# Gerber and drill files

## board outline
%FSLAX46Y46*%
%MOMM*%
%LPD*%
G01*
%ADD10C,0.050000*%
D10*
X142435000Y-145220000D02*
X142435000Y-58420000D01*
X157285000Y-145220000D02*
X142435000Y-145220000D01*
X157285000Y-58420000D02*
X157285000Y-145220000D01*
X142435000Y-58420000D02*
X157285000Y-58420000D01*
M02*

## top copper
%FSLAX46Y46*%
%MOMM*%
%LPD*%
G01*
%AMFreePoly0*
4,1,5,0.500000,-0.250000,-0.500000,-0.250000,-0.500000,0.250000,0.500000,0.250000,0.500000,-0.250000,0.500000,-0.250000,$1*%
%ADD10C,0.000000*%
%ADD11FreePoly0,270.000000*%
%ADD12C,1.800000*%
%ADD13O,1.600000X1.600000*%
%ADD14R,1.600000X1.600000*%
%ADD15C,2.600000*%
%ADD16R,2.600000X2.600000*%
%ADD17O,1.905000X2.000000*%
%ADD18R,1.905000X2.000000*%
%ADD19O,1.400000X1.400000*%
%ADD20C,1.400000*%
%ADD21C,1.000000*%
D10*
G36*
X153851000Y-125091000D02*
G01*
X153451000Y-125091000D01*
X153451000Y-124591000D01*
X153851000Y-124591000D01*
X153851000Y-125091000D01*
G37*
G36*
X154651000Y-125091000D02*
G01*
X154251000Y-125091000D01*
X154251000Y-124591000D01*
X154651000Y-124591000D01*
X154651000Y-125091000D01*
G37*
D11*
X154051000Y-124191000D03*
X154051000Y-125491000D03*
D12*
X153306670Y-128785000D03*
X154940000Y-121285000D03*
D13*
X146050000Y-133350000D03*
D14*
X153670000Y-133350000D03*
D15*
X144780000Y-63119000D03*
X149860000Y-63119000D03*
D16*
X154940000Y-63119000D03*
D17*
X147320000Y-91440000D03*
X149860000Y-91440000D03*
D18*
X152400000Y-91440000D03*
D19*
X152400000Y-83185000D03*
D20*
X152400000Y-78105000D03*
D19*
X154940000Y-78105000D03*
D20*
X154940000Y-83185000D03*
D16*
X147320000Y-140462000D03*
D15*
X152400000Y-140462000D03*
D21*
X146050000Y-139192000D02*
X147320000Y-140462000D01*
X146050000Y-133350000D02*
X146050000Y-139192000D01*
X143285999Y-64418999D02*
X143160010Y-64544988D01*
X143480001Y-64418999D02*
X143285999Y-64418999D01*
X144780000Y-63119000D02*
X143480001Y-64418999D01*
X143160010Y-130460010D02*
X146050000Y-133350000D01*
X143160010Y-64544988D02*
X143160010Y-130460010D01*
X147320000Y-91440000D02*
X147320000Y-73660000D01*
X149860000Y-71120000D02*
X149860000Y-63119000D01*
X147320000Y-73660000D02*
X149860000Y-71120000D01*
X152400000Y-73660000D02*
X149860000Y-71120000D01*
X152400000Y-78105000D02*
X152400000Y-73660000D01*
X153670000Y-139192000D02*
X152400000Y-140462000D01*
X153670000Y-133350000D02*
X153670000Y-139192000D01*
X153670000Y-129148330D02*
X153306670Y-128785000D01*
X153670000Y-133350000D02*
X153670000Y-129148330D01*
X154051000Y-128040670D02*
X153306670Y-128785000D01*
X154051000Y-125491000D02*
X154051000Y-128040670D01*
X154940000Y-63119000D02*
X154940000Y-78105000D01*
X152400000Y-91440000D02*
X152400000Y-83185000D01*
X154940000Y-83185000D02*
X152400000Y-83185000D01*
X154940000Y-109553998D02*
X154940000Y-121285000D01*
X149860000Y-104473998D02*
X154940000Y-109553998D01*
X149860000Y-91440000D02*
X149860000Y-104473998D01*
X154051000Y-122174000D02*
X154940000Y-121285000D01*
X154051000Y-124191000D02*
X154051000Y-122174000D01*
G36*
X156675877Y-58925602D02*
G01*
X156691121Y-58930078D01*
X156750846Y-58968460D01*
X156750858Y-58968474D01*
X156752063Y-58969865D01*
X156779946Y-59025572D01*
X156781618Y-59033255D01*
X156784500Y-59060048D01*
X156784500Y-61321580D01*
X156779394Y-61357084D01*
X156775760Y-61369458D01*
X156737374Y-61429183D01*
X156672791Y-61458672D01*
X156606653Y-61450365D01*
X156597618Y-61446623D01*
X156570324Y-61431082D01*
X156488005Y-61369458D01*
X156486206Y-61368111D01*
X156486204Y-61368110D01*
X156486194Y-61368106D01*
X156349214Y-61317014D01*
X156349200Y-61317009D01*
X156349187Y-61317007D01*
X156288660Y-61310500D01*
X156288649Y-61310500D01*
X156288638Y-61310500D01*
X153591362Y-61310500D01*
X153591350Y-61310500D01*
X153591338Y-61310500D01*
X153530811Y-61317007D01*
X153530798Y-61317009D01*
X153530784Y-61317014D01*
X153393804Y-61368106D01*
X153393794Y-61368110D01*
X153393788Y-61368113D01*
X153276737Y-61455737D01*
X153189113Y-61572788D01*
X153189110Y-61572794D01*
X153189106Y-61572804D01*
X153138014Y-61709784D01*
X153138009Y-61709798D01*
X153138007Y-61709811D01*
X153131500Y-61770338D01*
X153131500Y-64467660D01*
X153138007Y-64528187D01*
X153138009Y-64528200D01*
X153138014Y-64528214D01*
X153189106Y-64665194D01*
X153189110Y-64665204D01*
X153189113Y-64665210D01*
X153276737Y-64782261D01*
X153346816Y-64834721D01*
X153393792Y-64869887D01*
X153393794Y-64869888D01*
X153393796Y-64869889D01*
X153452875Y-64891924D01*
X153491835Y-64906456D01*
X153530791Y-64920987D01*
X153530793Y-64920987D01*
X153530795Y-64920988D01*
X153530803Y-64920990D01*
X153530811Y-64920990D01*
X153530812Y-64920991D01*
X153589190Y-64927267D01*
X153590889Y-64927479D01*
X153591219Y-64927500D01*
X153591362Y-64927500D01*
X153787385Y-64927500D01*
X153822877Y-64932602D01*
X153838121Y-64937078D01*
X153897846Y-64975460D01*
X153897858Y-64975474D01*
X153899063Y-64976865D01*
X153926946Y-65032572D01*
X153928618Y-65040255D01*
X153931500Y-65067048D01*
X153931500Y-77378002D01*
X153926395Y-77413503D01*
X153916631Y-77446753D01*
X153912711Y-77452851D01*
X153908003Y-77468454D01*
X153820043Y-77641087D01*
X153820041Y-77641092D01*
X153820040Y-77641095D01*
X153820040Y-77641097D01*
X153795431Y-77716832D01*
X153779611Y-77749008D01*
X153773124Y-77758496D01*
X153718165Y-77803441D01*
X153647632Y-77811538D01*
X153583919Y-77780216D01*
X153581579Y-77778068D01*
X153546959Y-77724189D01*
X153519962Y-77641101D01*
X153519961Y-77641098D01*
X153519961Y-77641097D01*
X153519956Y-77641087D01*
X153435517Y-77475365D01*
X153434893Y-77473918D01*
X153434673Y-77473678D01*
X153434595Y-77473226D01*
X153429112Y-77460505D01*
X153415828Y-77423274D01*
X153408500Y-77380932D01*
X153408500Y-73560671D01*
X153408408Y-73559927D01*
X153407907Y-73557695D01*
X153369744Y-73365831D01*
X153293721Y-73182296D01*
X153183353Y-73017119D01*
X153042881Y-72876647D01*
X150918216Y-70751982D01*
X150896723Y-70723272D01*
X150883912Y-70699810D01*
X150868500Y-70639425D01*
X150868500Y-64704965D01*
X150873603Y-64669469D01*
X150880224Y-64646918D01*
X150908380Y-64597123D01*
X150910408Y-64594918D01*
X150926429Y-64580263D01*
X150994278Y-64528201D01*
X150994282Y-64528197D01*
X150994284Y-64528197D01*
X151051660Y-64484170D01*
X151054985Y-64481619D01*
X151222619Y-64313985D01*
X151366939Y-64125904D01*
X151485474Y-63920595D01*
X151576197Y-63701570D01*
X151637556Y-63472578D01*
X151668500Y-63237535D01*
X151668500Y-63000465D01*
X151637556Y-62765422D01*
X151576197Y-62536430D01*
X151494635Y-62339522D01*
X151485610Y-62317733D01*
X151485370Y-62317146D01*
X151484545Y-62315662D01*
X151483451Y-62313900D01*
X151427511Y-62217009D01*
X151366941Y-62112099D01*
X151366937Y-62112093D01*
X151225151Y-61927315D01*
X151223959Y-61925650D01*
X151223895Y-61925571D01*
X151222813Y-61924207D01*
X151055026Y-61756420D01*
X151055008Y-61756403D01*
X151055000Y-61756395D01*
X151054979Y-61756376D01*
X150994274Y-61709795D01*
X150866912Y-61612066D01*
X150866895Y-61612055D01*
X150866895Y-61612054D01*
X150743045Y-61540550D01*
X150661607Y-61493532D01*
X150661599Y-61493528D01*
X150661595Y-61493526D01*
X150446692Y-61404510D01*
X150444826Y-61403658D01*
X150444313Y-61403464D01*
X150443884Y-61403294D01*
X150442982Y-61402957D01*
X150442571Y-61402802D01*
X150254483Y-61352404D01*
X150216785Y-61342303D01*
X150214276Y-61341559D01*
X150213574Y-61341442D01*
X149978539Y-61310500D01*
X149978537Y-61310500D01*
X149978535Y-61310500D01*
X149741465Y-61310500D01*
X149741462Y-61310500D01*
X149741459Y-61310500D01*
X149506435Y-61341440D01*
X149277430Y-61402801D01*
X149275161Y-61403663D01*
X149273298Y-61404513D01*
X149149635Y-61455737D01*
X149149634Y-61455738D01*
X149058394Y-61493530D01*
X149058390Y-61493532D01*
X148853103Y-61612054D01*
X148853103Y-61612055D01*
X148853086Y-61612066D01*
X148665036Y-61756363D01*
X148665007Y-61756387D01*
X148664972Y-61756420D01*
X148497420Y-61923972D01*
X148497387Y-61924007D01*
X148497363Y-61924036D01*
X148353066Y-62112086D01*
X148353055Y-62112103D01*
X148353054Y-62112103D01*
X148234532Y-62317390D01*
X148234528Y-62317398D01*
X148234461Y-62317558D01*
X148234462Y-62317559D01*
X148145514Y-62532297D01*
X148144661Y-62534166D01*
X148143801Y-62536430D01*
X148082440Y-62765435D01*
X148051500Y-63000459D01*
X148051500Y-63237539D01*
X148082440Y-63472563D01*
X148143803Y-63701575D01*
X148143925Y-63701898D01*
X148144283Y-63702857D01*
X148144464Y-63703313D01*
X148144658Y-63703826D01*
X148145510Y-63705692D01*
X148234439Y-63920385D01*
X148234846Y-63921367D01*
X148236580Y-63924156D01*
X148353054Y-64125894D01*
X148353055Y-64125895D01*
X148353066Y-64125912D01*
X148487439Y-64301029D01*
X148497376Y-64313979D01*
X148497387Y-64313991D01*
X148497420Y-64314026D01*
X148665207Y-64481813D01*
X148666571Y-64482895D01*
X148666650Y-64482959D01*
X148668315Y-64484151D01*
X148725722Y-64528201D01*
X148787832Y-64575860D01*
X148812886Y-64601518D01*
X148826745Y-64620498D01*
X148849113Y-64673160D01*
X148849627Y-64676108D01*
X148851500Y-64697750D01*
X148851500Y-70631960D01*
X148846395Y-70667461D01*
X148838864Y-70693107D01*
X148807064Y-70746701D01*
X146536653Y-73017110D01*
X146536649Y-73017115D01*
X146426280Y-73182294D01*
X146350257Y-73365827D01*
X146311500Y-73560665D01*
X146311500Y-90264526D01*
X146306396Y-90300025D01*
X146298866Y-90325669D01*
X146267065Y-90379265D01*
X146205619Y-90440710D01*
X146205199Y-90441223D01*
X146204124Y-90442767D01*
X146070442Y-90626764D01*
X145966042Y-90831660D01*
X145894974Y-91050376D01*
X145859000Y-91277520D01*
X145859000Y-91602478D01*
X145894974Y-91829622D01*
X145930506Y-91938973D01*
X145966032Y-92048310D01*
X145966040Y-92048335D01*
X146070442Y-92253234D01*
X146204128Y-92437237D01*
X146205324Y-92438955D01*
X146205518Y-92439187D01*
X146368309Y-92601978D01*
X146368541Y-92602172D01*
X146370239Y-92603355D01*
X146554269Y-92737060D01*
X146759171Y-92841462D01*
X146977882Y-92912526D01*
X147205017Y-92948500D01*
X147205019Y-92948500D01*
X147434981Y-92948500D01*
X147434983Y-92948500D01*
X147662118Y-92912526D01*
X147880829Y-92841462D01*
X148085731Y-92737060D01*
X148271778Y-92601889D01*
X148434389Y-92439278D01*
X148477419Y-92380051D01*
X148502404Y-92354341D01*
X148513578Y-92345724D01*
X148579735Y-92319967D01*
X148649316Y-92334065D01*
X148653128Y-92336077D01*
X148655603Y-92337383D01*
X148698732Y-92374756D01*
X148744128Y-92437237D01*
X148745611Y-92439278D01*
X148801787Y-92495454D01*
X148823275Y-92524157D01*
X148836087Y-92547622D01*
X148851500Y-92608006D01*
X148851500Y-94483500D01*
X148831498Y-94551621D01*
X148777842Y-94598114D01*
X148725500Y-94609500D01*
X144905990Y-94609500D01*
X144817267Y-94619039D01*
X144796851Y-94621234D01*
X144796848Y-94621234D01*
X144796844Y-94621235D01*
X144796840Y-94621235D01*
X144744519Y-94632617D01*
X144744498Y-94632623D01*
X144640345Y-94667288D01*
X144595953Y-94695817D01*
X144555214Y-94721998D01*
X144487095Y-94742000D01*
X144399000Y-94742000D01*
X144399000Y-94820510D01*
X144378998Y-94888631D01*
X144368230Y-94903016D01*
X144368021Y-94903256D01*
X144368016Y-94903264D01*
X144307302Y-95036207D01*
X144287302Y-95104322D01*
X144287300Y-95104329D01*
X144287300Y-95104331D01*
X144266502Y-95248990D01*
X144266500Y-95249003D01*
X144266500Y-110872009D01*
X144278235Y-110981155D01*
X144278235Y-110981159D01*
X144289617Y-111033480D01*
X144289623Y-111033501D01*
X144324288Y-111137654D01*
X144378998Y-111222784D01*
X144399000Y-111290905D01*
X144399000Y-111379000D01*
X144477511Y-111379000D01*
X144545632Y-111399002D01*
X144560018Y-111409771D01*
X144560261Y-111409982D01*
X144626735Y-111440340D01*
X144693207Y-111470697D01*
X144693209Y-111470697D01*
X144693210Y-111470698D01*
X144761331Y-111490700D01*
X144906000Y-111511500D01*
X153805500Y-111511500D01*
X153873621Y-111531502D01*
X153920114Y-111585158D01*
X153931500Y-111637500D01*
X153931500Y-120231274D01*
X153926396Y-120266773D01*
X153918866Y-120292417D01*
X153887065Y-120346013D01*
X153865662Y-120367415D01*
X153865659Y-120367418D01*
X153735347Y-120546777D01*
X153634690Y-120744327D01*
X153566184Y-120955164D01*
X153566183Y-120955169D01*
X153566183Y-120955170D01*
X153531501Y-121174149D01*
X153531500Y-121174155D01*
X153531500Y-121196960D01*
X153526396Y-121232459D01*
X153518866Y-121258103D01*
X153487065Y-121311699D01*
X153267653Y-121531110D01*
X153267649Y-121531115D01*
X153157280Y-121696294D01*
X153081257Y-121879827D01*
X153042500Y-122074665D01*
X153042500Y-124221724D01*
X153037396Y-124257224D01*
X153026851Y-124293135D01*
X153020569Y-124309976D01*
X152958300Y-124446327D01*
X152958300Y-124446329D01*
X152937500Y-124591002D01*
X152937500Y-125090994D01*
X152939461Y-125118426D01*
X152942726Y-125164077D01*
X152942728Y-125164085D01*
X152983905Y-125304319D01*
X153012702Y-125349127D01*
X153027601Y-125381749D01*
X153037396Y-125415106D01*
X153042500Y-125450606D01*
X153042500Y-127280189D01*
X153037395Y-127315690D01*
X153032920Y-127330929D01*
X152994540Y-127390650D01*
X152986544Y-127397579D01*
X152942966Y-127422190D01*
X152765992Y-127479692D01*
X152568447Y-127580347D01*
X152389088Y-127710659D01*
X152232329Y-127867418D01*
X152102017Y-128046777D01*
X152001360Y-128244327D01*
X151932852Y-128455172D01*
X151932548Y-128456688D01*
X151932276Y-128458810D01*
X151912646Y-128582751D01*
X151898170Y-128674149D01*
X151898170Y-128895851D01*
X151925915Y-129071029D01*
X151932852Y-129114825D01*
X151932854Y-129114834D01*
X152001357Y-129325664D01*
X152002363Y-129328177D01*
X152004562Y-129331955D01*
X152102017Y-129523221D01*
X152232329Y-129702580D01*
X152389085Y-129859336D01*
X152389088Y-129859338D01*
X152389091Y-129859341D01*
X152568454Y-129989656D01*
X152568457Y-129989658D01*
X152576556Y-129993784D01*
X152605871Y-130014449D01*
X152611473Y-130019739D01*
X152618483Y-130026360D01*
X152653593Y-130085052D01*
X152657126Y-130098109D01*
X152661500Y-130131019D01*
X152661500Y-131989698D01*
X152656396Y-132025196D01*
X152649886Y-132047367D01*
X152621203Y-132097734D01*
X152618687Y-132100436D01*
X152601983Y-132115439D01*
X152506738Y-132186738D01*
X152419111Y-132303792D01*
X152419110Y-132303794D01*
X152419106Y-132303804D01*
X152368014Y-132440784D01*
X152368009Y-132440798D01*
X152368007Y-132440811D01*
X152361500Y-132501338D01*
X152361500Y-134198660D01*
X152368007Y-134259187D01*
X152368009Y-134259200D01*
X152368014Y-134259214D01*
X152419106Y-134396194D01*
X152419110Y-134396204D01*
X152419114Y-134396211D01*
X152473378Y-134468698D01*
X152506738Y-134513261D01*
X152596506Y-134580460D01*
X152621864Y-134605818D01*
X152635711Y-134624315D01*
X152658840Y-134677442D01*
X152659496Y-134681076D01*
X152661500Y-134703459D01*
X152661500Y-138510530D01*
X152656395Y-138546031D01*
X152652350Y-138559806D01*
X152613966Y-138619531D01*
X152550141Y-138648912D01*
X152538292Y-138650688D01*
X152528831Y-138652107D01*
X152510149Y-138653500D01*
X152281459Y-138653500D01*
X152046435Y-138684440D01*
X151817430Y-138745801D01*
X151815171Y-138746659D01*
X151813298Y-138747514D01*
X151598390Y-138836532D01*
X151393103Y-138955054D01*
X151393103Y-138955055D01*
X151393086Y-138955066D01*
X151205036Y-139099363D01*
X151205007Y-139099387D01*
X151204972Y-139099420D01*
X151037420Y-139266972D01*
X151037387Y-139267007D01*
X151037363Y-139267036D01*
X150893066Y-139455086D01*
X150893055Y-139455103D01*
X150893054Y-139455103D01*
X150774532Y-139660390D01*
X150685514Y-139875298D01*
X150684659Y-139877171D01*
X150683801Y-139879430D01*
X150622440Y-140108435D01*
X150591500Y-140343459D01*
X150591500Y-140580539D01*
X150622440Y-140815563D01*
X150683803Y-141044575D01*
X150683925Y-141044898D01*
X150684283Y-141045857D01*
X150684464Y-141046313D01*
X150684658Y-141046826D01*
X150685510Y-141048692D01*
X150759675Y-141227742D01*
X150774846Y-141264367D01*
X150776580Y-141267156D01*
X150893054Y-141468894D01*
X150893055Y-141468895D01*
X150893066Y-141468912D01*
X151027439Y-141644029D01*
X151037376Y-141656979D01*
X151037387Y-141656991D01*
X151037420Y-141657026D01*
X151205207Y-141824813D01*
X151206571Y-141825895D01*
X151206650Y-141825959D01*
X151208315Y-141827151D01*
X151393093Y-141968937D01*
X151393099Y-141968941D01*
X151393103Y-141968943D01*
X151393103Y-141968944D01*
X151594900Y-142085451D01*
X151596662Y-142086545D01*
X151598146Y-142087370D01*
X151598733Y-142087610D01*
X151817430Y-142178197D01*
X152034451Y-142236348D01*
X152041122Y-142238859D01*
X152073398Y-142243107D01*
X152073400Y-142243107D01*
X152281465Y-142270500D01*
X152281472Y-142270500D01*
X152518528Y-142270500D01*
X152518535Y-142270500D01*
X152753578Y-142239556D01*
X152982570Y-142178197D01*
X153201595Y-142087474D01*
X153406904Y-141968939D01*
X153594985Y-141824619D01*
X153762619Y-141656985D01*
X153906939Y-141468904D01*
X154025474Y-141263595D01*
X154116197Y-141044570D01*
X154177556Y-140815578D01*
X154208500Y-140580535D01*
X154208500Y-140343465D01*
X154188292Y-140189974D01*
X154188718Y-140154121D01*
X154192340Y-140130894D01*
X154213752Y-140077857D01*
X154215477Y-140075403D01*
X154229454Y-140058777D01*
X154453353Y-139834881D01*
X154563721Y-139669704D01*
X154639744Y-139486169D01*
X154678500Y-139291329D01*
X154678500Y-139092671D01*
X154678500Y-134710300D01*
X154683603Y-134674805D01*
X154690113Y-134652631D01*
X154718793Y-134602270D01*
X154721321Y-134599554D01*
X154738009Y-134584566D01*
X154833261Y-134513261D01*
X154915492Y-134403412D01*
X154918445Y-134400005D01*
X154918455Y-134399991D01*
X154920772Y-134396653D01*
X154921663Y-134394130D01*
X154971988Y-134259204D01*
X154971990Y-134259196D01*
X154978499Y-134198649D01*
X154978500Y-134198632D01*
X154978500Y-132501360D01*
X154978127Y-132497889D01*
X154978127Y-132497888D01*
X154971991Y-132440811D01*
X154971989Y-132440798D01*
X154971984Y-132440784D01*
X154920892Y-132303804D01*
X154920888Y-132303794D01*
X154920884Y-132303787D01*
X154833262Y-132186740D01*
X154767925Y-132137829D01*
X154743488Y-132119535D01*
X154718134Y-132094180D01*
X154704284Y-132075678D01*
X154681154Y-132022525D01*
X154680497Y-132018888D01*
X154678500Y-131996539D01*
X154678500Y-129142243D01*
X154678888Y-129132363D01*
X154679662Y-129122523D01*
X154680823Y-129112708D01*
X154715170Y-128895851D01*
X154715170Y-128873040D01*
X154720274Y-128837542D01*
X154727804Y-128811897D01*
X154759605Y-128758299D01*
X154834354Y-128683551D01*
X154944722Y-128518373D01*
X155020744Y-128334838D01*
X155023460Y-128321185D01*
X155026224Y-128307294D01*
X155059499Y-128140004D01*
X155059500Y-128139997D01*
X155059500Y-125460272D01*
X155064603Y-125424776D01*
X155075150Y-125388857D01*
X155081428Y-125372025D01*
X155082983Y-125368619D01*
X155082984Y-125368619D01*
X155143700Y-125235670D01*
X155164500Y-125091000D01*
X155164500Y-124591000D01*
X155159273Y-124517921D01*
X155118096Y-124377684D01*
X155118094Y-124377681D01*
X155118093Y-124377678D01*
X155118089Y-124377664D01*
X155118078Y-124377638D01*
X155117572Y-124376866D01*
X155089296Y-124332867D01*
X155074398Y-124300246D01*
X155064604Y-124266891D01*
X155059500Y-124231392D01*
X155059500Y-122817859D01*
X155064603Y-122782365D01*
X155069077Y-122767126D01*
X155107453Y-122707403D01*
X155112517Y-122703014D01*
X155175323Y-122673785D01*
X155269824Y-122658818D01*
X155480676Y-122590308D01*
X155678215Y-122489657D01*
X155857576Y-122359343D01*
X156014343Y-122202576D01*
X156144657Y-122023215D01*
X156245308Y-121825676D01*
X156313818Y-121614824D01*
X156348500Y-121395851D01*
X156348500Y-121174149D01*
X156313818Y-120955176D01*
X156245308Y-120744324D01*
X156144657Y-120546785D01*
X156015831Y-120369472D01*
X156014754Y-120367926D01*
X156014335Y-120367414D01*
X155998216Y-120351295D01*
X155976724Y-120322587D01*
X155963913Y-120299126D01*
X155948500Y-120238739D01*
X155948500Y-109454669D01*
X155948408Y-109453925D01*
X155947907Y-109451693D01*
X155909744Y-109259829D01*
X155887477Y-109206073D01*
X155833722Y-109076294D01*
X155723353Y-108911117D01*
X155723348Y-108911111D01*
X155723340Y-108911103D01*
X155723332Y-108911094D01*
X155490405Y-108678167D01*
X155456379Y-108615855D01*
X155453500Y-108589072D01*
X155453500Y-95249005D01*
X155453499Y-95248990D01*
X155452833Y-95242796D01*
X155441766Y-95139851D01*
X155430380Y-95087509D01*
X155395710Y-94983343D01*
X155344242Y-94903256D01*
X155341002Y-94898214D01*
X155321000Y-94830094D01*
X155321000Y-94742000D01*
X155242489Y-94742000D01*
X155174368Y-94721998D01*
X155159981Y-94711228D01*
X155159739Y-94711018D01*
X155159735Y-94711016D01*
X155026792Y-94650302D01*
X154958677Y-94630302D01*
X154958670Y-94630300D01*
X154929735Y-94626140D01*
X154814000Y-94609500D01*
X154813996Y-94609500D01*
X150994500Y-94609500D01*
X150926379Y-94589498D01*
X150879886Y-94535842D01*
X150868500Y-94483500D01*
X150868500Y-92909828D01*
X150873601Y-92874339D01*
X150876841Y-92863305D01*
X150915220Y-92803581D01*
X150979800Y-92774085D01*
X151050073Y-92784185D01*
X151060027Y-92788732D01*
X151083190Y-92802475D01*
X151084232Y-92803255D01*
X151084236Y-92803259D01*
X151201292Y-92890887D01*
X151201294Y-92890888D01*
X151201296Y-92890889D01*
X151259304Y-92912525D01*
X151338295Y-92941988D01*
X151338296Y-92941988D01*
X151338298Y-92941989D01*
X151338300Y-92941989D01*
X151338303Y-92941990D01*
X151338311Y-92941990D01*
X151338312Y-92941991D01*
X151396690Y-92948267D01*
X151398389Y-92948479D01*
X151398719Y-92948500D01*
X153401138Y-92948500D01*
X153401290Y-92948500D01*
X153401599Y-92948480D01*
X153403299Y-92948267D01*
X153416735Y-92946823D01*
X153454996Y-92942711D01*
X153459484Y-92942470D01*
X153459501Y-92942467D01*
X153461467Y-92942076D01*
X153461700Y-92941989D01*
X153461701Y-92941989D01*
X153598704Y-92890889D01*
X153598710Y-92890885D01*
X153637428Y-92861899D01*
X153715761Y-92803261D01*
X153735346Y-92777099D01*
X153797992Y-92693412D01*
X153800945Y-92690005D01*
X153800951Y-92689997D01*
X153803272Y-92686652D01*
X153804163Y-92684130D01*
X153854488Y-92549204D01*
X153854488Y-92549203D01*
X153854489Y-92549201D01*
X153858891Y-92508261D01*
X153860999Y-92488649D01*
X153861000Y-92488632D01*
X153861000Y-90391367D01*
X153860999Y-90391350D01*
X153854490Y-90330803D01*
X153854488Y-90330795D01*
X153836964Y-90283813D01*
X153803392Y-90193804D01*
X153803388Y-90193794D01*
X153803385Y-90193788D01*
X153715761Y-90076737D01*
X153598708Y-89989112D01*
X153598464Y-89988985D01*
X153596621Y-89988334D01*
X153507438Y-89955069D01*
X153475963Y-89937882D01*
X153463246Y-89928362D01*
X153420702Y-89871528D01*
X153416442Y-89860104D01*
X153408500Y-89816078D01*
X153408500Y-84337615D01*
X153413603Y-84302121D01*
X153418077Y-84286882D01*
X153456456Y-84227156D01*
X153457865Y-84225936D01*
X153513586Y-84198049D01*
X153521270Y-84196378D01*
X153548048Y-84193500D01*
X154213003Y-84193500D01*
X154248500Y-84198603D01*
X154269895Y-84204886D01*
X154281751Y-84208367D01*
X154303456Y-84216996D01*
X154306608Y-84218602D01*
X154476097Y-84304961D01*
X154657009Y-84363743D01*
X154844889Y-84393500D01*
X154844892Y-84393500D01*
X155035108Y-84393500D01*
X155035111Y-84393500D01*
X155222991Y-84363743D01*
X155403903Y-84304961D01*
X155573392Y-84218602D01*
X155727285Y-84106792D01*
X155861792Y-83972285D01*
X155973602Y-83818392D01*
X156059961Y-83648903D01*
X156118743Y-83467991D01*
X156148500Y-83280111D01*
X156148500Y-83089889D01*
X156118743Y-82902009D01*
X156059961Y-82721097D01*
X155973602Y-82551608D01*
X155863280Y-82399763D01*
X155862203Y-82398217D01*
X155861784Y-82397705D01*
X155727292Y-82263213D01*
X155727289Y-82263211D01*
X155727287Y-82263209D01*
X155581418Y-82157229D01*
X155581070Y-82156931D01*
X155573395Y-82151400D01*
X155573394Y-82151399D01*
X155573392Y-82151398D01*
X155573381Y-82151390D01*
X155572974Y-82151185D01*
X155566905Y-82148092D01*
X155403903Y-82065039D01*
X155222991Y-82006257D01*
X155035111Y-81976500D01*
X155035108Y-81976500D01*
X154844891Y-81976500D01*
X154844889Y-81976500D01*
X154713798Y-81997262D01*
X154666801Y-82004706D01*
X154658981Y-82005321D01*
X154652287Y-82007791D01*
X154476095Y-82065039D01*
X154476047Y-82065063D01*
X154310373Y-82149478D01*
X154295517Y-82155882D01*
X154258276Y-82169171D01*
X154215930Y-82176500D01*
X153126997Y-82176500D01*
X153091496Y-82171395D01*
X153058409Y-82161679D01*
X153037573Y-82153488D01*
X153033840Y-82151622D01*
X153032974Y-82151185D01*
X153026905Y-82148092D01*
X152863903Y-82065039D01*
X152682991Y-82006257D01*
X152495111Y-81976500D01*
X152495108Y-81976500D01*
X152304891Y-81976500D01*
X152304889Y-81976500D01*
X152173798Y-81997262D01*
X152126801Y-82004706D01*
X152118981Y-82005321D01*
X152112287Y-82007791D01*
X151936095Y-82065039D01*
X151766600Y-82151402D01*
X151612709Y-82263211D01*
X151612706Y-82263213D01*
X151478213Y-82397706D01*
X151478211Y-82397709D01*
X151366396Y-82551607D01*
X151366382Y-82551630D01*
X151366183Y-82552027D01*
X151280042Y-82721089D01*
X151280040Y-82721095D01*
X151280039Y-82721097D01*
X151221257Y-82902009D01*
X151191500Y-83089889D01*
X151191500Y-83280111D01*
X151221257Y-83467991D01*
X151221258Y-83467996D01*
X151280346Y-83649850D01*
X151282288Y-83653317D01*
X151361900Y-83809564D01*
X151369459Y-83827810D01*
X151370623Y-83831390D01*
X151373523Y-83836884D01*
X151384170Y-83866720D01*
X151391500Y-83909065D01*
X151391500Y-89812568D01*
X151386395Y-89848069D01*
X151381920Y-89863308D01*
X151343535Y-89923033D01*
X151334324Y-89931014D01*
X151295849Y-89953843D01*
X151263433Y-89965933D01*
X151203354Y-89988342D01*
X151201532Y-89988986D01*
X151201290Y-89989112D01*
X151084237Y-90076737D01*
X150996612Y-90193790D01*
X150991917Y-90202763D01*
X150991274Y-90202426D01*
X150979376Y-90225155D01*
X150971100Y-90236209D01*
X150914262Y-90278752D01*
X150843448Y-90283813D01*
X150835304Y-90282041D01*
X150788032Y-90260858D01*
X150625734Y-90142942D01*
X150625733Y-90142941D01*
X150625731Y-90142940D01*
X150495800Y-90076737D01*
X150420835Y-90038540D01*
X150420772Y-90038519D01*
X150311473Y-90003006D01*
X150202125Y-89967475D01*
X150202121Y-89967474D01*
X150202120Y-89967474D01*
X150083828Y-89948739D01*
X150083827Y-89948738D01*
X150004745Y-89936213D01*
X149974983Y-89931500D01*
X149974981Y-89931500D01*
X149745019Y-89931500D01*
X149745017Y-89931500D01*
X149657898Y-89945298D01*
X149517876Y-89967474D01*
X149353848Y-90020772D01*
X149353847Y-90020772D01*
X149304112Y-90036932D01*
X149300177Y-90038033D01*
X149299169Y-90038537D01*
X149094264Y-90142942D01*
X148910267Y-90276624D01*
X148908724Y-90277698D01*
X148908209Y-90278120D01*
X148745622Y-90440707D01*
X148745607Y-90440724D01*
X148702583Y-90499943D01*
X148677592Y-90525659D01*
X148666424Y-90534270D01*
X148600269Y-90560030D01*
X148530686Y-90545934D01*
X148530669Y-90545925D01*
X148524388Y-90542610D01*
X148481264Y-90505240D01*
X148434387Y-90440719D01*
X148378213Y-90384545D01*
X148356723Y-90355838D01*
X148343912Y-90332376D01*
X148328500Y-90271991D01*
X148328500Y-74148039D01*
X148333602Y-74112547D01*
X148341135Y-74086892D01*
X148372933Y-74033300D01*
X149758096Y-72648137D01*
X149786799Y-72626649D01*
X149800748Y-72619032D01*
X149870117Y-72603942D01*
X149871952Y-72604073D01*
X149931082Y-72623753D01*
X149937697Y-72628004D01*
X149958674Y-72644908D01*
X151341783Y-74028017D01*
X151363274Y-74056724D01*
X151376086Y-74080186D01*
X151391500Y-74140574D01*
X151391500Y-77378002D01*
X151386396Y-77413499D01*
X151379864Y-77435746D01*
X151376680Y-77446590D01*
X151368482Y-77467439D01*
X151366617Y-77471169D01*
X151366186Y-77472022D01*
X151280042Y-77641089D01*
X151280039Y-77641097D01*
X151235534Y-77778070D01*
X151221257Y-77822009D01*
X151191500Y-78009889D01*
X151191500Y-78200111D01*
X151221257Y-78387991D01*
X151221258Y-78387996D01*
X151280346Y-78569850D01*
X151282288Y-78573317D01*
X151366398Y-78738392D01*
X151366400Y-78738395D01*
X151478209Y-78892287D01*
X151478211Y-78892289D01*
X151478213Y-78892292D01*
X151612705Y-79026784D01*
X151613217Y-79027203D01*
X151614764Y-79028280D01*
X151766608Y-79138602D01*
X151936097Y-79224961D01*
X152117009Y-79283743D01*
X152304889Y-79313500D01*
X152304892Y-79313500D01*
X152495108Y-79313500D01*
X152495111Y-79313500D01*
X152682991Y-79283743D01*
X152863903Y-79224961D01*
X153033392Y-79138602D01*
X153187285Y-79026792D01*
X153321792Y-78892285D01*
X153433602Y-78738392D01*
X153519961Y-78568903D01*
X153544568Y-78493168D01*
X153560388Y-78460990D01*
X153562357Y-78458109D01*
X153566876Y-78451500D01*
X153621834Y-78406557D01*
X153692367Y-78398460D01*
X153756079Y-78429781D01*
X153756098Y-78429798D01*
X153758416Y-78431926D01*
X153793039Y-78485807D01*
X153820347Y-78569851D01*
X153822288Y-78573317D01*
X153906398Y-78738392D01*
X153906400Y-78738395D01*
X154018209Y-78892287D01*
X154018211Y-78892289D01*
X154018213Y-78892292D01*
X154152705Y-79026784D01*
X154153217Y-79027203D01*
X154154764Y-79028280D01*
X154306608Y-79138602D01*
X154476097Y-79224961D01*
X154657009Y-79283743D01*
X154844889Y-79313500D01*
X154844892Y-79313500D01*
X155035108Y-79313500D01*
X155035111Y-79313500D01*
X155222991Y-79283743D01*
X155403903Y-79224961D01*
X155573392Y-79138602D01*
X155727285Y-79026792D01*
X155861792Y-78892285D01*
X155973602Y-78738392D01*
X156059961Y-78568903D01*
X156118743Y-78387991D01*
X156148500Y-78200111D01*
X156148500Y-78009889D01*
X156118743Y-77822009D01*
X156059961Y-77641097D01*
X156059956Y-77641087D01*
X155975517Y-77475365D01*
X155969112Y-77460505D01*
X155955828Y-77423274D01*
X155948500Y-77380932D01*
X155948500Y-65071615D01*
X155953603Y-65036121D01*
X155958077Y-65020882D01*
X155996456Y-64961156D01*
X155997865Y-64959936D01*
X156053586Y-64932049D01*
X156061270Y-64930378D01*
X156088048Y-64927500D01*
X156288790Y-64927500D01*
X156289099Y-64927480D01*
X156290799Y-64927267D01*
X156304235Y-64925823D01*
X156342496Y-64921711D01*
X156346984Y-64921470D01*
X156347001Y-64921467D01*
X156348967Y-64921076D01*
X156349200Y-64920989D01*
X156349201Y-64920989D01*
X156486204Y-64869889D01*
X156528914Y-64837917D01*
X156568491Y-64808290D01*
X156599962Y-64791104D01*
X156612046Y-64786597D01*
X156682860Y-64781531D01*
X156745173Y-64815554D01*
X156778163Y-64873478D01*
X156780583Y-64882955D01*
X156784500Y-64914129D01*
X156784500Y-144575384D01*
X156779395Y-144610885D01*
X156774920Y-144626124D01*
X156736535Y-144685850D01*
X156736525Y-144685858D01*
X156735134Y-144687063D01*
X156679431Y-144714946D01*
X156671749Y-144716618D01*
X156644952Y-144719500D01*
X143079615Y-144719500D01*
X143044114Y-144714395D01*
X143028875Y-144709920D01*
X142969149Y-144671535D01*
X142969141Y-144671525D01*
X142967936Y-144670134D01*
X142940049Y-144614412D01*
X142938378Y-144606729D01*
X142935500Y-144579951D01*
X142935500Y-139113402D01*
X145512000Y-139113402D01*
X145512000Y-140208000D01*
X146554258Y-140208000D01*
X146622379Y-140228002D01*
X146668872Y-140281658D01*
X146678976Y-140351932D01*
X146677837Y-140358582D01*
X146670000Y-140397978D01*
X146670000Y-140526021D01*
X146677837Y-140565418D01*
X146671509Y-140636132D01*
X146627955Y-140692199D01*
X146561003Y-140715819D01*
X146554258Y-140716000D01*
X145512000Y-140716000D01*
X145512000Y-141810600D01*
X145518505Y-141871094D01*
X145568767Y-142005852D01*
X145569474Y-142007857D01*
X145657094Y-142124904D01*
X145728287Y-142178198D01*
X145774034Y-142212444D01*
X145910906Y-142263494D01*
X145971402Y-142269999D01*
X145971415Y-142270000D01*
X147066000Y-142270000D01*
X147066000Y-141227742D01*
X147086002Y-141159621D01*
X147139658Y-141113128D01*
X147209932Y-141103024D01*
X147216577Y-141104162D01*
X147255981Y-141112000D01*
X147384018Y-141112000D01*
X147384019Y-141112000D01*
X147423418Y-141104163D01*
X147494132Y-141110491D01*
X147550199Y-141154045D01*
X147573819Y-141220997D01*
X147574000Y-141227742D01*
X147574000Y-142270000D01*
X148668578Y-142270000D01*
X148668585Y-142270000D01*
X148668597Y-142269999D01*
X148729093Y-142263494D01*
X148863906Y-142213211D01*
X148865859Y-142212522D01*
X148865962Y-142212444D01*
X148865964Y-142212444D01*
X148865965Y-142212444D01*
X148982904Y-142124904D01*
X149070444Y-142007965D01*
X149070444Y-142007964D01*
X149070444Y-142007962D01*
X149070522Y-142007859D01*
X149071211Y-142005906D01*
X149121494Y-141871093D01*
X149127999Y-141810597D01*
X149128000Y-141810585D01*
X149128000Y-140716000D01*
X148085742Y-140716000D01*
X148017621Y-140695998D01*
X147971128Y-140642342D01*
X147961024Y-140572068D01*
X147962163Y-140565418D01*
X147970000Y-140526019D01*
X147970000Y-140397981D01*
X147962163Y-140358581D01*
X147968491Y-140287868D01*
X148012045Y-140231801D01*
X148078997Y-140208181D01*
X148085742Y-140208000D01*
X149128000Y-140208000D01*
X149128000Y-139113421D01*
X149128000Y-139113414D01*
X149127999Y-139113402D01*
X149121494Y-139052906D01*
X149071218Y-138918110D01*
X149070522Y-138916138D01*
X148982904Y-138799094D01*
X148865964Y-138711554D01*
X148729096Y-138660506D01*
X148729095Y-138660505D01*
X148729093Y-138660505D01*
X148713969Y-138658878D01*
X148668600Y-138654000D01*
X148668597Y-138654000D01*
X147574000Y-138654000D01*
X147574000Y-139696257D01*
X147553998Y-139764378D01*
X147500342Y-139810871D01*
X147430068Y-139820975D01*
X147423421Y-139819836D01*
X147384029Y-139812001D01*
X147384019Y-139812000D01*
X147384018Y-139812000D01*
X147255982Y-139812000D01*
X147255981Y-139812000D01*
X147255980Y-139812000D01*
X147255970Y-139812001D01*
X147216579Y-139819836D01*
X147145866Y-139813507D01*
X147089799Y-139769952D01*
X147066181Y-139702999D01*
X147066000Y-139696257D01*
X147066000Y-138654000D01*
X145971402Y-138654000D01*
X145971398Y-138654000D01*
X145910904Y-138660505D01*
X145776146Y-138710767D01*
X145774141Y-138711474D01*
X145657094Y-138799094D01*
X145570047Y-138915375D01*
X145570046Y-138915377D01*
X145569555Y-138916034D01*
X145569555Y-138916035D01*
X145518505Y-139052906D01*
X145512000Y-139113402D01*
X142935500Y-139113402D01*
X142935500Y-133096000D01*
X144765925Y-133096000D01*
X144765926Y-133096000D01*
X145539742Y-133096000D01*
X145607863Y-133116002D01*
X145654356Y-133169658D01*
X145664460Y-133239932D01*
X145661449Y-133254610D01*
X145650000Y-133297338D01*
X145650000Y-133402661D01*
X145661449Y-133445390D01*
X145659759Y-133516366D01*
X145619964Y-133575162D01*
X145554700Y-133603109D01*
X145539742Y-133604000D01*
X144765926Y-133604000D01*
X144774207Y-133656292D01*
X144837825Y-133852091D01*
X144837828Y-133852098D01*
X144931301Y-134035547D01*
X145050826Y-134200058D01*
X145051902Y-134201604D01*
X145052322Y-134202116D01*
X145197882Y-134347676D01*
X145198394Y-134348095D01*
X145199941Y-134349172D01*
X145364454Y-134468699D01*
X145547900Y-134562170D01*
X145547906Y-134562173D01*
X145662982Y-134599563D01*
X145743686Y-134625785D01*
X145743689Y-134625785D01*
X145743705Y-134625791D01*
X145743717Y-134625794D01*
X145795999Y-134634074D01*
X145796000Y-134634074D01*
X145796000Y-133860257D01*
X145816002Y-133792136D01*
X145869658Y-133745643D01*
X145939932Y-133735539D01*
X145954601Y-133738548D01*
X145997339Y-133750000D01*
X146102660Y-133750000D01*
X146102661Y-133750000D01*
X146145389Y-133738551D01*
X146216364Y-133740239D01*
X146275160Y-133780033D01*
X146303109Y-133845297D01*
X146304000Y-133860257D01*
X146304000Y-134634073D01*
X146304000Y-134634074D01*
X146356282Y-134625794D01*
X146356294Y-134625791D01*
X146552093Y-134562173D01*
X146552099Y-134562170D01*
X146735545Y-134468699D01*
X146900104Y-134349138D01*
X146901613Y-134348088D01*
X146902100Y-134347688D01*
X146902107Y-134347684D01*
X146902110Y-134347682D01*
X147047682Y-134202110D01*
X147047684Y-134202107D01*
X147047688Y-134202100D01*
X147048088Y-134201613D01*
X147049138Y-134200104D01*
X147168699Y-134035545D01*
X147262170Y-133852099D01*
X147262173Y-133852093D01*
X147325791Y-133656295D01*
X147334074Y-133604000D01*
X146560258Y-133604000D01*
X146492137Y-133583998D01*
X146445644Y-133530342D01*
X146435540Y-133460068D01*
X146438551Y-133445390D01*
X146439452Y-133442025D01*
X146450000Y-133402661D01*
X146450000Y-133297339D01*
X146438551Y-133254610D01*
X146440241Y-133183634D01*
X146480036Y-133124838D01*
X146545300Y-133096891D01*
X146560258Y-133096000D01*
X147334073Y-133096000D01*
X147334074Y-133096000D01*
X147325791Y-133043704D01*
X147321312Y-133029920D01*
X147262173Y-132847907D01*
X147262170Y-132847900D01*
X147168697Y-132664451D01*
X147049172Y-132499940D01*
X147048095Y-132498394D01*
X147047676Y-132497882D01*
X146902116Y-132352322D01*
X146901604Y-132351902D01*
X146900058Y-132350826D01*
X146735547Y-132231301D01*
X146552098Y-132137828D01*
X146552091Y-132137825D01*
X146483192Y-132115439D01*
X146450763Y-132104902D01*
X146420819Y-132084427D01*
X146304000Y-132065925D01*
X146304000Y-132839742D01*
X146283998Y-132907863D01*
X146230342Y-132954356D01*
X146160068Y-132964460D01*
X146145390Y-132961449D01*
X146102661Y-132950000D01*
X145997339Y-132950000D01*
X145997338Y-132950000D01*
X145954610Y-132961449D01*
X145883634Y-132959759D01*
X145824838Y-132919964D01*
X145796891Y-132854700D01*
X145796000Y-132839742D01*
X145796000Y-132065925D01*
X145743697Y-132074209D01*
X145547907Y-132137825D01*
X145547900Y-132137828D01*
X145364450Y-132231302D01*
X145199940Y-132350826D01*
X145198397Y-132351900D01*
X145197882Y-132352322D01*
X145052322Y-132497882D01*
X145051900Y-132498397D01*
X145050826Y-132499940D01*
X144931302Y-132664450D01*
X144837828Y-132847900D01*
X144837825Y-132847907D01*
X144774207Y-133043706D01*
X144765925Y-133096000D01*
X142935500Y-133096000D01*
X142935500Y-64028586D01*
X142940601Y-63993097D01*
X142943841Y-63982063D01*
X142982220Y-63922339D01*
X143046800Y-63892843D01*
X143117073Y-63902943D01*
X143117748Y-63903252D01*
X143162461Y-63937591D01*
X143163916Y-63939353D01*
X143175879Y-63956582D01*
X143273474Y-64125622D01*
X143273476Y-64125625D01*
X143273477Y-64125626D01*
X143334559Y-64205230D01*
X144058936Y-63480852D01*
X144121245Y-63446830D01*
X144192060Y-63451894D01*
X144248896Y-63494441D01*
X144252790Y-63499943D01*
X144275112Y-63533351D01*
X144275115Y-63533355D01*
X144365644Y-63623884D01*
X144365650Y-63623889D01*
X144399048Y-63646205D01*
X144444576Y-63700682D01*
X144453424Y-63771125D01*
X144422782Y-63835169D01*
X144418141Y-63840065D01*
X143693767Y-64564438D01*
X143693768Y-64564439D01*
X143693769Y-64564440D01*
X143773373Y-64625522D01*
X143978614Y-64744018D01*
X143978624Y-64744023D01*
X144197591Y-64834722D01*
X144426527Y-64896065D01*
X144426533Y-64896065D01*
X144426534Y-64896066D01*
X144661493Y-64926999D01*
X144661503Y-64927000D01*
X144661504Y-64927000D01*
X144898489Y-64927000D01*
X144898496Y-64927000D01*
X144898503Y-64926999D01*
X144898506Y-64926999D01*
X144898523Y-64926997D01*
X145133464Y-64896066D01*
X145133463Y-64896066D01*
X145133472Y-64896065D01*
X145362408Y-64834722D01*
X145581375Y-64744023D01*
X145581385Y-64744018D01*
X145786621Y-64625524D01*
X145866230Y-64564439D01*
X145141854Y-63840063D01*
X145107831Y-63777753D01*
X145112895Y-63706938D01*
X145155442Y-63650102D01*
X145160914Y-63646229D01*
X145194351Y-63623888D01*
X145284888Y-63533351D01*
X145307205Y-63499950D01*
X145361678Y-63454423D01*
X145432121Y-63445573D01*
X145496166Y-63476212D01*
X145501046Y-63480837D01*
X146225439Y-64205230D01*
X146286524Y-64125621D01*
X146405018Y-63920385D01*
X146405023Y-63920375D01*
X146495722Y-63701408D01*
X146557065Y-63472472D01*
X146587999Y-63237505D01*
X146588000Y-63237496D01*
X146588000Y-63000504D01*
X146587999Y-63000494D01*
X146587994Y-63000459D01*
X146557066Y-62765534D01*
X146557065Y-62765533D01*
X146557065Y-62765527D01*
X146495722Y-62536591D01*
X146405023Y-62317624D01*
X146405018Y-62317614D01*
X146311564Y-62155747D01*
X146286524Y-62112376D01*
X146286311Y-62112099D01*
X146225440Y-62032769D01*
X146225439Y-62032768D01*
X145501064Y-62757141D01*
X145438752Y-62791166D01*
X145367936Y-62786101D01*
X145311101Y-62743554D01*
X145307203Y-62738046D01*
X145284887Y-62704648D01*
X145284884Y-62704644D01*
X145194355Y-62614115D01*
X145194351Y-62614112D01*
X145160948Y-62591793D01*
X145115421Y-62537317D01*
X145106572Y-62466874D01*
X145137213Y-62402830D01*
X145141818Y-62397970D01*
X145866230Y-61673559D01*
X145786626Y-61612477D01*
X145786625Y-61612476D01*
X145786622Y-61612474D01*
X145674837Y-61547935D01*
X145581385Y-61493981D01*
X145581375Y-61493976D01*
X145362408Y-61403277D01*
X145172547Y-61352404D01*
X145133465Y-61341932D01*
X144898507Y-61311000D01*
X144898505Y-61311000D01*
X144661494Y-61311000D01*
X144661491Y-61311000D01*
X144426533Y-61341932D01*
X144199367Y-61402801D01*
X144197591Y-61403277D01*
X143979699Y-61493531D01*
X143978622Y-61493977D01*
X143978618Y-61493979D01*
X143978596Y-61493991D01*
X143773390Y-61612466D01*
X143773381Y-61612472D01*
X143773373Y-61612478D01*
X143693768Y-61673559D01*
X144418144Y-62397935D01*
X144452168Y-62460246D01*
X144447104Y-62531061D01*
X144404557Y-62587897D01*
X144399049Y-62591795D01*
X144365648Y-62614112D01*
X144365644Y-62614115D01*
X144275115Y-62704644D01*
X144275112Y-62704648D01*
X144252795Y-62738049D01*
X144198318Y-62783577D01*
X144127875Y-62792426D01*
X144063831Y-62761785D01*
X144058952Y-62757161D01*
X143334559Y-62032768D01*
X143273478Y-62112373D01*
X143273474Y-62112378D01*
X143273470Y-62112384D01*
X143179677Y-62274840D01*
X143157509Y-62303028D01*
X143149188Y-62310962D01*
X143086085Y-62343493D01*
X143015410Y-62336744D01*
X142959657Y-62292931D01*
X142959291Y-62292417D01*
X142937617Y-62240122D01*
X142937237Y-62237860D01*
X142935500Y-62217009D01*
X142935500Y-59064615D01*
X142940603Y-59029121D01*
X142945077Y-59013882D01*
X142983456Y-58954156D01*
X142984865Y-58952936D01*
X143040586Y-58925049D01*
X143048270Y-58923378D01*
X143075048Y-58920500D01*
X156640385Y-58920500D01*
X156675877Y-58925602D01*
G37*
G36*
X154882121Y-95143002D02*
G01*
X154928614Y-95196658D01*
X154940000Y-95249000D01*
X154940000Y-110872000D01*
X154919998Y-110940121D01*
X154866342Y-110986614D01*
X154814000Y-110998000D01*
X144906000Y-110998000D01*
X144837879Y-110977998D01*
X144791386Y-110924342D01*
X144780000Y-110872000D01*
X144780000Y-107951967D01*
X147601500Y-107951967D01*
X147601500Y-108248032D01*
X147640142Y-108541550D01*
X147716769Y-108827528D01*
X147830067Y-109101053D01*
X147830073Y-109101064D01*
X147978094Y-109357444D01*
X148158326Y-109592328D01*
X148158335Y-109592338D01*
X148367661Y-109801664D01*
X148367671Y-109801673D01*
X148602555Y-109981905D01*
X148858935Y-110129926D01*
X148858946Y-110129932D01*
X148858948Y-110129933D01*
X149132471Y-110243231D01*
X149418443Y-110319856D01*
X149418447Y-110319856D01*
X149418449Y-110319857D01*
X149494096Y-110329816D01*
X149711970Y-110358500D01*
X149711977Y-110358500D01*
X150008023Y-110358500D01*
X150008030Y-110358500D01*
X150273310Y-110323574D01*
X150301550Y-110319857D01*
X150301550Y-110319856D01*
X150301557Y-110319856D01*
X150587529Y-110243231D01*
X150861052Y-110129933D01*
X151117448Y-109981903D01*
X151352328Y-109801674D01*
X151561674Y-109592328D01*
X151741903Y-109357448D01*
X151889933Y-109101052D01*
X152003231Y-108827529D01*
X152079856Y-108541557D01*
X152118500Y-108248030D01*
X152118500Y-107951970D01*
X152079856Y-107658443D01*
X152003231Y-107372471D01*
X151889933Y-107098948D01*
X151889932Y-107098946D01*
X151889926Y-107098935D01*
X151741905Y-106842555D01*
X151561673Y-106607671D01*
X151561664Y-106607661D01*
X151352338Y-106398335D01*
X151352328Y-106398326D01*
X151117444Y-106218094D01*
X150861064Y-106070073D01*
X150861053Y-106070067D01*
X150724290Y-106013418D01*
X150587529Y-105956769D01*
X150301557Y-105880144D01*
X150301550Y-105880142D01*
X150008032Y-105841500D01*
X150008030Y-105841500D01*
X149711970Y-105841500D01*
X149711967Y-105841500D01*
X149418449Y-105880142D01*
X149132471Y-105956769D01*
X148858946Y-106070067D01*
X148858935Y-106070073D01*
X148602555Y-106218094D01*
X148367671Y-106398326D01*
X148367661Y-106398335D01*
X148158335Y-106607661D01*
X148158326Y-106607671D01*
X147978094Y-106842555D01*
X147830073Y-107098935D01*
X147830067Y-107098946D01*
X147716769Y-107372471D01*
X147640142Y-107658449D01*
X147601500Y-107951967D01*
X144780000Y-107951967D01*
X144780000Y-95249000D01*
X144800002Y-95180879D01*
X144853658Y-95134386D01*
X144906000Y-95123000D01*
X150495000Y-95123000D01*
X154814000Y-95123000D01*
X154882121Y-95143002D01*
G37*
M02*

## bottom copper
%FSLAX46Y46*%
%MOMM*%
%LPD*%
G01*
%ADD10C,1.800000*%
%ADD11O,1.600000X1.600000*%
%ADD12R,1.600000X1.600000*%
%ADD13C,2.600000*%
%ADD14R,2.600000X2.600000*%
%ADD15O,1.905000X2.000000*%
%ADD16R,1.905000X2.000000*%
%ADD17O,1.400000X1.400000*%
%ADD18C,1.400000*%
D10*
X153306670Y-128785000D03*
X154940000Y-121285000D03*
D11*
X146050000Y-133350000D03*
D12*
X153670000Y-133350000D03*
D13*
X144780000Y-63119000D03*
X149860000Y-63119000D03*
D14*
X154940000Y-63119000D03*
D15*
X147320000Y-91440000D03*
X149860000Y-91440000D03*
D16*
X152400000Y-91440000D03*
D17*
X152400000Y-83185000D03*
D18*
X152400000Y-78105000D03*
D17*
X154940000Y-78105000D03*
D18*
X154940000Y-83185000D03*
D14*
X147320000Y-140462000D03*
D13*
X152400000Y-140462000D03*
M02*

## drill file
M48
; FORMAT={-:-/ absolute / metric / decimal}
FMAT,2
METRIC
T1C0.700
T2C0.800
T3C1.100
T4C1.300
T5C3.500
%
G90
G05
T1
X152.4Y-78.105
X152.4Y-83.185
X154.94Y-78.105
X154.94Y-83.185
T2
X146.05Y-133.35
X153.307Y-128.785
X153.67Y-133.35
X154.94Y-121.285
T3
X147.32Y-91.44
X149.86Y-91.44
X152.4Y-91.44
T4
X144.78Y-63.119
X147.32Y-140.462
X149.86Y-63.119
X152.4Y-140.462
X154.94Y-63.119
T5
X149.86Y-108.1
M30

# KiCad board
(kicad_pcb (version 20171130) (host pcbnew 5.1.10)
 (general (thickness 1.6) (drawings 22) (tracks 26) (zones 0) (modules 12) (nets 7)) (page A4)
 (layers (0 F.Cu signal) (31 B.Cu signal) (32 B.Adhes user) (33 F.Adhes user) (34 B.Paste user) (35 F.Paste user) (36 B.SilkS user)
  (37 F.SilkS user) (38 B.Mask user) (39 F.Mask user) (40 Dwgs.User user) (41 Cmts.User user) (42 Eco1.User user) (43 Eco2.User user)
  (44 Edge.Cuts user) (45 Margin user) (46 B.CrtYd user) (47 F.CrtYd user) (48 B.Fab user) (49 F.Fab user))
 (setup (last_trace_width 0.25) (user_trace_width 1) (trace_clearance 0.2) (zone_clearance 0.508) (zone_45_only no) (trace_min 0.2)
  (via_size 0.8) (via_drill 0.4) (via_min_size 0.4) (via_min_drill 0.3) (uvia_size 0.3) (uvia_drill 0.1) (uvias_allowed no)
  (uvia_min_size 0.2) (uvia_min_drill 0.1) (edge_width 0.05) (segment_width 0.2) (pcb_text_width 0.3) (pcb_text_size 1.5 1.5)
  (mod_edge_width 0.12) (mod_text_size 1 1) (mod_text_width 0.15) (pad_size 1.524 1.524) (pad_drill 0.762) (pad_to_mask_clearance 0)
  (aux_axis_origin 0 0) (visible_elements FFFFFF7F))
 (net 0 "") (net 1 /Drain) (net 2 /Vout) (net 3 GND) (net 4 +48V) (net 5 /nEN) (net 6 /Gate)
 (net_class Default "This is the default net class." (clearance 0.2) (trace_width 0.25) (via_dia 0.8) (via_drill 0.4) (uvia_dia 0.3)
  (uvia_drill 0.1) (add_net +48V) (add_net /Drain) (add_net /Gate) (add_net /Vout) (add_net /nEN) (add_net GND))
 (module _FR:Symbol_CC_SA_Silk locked (layer B.Cu) (at 146.304 86.487 180)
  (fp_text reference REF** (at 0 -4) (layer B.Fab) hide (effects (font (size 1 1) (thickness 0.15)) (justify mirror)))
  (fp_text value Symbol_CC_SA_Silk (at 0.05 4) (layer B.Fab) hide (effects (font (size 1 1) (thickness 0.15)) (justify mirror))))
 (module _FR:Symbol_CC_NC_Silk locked (layer B.Cu) (at 146.304 79.375 180)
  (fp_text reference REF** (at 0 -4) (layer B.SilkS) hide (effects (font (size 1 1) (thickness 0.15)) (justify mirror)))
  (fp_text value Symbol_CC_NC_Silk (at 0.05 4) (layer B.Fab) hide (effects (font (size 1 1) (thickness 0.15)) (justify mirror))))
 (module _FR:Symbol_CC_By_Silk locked (layer B.Cu) (at 146.304 72.39 180)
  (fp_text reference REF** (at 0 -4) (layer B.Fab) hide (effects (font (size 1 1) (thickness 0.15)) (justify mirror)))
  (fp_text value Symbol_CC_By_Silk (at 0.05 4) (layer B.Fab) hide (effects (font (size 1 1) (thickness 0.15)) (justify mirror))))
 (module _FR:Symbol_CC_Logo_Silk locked (layer B.Cu) (at 153.289 72.263 180)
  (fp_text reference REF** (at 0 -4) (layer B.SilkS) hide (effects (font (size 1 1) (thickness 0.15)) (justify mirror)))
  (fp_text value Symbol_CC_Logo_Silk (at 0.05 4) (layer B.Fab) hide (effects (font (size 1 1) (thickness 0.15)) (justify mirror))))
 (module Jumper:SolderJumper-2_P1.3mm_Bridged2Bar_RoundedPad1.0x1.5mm (layer F.Cu) (at 154.051 124.841 270)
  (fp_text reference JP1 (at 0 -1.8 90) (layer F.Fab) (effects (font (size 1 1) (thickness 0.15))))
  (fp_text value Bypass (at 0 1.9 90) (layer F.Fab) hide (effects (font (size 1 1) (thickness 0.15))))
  (fp_poly (pts (xy -0.25 0.2) (xy 0.25 0.2) (xy 0.25 0.6) (xy -0.25 0.6)) (layer F.Cu) (width 0))
  (fp_poly (pts (xy -0.25 -0.6) (xy 0.25 -0.6) (xy 0.25 -0.2) (xy -0.25 -0.2)) (layer F.Cu) (width 0))
  (pad 1 smd custom (at -0.65 0 270) (size 1 0.5) (layers F.Cu F.Mask) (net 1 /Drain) (zone_connect 2)
   (options (clearance outline) (anchor rect)) (primitives))
  (pad 2 smd custom (at 0.65 0 270) (size 1 0.5) (layers F.Cu F.Mask) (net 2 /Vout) (zone_connect 2)
   (options (clearance outline) (anchor rect)) (primitives)))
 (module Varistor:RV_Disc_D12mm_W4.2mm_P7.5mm (layer F.Cu) (at 154.94 121.285 270)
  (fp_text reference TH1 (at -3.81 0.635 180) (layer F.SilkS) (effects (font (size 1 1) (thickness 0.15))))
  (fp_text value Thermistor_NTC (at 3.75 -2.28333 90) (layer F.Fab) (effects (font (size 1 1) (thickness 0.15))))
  (pad 2 thru_hole circle (at 7.5 1.63333 270) (size 1.8 1.8) (drill 0.8) (layers *.Cu *.Mask) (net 2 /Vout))
  (pad 1 thru_hole circle (at 0 0 270) (size 1.8 1.8) (drill 0.8) (layers *.Cu *.Mask) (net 1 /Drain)))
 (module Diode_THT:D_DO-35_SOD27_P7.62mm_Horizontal (layer F.Cu) (at 153.67 133.35 180)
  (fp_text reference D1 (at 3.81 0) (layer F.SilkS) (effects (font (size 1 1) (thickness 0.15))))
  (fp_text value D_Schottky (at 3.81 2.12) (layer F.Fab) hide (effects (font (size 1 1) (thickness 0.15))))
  (pad 2 thru_hole oval (at 7.62 0 180) (size 1.6 1.6) (drill 0.8) (layers *.Cu *.Mask) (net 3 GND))
  (pad 1 thru_hole rect (at 0 0 180) (size 1.6 1.6) (drill 0.8) (layers *.Cu *.Mask) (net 2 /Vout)))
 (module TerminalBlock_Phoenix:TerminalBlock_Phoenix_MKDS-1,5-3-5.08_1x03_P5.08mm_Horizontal (layer F.Cu) (at 154.94 63.119 180)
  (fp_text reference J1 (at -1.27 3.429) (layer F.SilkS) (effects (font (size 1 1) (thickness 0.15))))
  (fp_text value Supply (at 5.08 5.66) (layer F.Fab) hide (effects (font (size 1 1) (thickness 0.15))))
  (pad 3 thru_hole circle (at 10.16 0 180) (size 2.6 2.6) (drill 1.3) (layers *.Cu *.Mask) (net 3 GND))
  (pad 2 thru_hole circle (at 5.08 0 180) (size 2.6 2.6) (drill 1.3) (layers *.Cu *.Mask) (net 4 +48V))
  (pad 1 thru_hole rect (at 0 0 180) (size 2.6 2.6) (drill 1.3) (layers *.Cu *.Mask) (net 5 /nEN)))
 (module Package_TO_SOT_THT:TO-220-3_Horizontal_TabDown (layer F.Cu) (at 152.4 91.44 180)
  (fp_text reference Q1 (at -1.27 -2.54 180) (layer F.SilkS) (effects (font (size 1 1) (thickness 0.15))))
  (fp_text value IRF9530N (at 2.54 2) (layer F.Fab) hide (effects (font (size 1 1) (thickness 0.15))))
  (pad 3 thru_hole oval (at 5.08 0 180) (size 1.905 2) (drill 1.1) (layers *.Cu *.Mask) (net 4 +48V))
  (pad 2 thru_hole oval (at 2.54 0 180) (size 1.905 2) (drill 1.1) (layers *.Cu *.Mask) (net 1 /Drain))
  (pad 1 thru_hole rect (at 0 0 180) (size 1.905 2) (drill 1.1) (layers *.Cu *.Mask) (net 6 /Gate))
  (pad "" np_thru_hole oval (at 2.54 -16.66 180) (size 3.5 3.5) (drill 3.5) (layers *.Cu *.Mask)))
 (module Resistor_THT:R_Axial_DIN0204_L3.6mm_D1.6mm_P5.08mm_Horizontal (layer F.Cu) (at 152.4 78.105 270)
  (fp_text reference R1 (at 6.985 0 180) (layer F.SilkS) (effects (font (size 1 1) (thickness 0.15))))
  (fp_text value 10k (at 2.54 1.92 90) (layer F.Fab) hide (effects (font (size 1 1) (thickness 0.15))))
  (pad 2 thru_hole oval (at 5.08 0 270) (size 1.4 1.4) (drill 0.7) (layers *.Cu *.Mask) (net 6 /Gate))
  (pad 1 thru_hole circle (at 0 0 270) (size 1.4 1.4) (drill 0.7) (layers *.Cu *.Mask) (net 4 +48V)))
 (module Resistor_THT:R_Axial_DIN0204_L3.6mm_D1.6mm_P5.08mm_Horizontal (layer F.Cu) (at 154.94 83.185 90)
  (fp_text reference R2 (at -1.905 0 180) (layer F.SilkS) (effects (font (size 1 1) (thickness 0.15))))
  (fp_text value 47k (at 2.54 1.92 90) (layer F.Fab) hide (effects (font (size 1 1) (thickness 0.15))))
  (pad 2 thru_hole oval (at 5.08 0 90) (size 1.4 1.4) (drill 0.7) (layers *.Cu *.Mask) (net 5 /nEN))
  (pad 1 thru_hole circle (at 0 0 90) (size 1.4 1.4) (drill 0.7) (layers *.Cu *.Mask) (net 6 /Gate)))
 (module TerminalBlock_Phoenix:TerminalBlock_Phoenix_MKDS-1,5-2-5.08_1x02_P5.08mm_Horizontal (layer F.Cu) (at 147.32 140.462)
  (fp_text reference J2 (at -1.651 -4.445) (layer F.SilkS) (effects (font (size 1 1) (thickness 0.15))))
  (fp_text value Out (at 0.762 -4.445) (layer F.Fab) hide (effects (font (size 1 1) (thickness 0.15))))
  (pad 1 thru_hole rect (at 0 0) (size 2.6 2.6) (drill 1.3) (layers *.Cu *.Mask) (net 3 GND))
  (pad 2 thru_hole circle (at 5.08 0) (size 2.6 2.6) (drill 1.3) (layers *.Cu *.Mask) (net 2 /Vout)))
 (gr_line (start 142.435 145.22) (end 142.435 58.42) (layer Edge.Cuts) (width 0.05))
 (gr_line (start 157.285 145.22) (end 142.435 145.22) (layer Edge.Cuts) (width 0.05))
 (gr_line (start 157.285 58.42) (end 157.285 145.22) (layer Edge.Cuts) (width 0.05))
 (gr_line (start 142.435 58.42) (end 157.285 58.42) (layer Edge.Cuts) (width 0.05))
 (segment (start 146.05 139.192) (end 147.32 140.462) (width 1) (layer F.Cu) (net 3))
 (segment (start 146.05 133.35) (end 146.05 139.192) (width 1) (layer F.Cu) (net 3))
 (segment (start 143.285999 64.418999) (end 143.16001 64.544988) (width 1) (layer F.Cu) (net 3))
 (segment (start 143.480001 64.418999) (end 143.285999 64.418999) (width 1) (layer F.Cu) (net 3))
 (segment (start 144.78 63.119) (end 143.480001 64.418999) (width 1) (layer F.Cu) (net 3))
 (segment (start 143.16001 130.46001) (end 146.05 133.35) (width 1) (layer F.Cu) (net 3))
 (segment (start 143.16001 64.544988) (end 143.16001 130.46001) (width 1) (layer F.Cu) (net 3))
 (segment (start 147.32 91.44) (end 147.32 73.66) (width 1) (layer F.Cu) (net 4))
 (segment (start 149.86 71.12) (end 149.86 63.119) (width 1) (layer F.Cu) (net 4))
 (segment (start 147.32 73.66) (end 149.86 71.12) (width 1) (layer F.Cu) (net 4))
 (segment (start 152.4 73.66) (end 149.86 71.12) (width 1) (layer F.Cu) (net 4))
 (segment (start 152.4 78.105) (end 152.4 73.66) (width 1) (layer F.Cu) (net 4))
 (segment (start 153.67 139.192) (end 152.4 140.462) (width 1) (layer F.Cu) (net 2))
 (segment (start 153.67 133.35) (end 153.67 139.192) (width 1) (layer F.Cu) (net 2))
 (segment (start 153.67 129.14833) (end 153.30667 128.785) (width 1) (layer F.Cu) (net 2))
 (segment (start 153.67 133.35) (end 153.67 129.14833) (width 1) (layer F.Cu) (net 2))
 (segment (start 154.051 128.04067) (end 153.30667 128.785) (width 1) (layer F.Cu) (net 2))
 (segment (start 154.051 125.491) (end 154.051 128.04067) (width 1) (layer F.Cu) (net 2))
 (segment (start 154.94 63.119) (end 154.94 78.105) (width 1) (layer F.Cu) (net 5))
 (segment (start 152.4 91.44) (end 152.4 83.185) (width 1) (layer F.Cu) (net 6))
 (segment (start 154.94 83.185) (end 152.4 83.185) (width 1) (layer F.Cu) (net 6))
 (segment (start 154.94 109.553998) (end 154.94 121.285) (width 1) (layer F.Cu) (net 1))
 (segment (start 149.86 104.473998) (end 154.94 109.553998) (width 1) (layer F.Cu) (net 1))
 (segment (start 149.86 91.44) (end 149.86 104.473998) (width 1) (layer F.Cu) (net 1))
 (segment (start 154.051 122.174) (end 154.94 121.285) (width 1) (layer F.Cu) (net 1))
 (segment (start 154.051 124.191) (end 154.051 122.174) (width 1) (layer F.Cu) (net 1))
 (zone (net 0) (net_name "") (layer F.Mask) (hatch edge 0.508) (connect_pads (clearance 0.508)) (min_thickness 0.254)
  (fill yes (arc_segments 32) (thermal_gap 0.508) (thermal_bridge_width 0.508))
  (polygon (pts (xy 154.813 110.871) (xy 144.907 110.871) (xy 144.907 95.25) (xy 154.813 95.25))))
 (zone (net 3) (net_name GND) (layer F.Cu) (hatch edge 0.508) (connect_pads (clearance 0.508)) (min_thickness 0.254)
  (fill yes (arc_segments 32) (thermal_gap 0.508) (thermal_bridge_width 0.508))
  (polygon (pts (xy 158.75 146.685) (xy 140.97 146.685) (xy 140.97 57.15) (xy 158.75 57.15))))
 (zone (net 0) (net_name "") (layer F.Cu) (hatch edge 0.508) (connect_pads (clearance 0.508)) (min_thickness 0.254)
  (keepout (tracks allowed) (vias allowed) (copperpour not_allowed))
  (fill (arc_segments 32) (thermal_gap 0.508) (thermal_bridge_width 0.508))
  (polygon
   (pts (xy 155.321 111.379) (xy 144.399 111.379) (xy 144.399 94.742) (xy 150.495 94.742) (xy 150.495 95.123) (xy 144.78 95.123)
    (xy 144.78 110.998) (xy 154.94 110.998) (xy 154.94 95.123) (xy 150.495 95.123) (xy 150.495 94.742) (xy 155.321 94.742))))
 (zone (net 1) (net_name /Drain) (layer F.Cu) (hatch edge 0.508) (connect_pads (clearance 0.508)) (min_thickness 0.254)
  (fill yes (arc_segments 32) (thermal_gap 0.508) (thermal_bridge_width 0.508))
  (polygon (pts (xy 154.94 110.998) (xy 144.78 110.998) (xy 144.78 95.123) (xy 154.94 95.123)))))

